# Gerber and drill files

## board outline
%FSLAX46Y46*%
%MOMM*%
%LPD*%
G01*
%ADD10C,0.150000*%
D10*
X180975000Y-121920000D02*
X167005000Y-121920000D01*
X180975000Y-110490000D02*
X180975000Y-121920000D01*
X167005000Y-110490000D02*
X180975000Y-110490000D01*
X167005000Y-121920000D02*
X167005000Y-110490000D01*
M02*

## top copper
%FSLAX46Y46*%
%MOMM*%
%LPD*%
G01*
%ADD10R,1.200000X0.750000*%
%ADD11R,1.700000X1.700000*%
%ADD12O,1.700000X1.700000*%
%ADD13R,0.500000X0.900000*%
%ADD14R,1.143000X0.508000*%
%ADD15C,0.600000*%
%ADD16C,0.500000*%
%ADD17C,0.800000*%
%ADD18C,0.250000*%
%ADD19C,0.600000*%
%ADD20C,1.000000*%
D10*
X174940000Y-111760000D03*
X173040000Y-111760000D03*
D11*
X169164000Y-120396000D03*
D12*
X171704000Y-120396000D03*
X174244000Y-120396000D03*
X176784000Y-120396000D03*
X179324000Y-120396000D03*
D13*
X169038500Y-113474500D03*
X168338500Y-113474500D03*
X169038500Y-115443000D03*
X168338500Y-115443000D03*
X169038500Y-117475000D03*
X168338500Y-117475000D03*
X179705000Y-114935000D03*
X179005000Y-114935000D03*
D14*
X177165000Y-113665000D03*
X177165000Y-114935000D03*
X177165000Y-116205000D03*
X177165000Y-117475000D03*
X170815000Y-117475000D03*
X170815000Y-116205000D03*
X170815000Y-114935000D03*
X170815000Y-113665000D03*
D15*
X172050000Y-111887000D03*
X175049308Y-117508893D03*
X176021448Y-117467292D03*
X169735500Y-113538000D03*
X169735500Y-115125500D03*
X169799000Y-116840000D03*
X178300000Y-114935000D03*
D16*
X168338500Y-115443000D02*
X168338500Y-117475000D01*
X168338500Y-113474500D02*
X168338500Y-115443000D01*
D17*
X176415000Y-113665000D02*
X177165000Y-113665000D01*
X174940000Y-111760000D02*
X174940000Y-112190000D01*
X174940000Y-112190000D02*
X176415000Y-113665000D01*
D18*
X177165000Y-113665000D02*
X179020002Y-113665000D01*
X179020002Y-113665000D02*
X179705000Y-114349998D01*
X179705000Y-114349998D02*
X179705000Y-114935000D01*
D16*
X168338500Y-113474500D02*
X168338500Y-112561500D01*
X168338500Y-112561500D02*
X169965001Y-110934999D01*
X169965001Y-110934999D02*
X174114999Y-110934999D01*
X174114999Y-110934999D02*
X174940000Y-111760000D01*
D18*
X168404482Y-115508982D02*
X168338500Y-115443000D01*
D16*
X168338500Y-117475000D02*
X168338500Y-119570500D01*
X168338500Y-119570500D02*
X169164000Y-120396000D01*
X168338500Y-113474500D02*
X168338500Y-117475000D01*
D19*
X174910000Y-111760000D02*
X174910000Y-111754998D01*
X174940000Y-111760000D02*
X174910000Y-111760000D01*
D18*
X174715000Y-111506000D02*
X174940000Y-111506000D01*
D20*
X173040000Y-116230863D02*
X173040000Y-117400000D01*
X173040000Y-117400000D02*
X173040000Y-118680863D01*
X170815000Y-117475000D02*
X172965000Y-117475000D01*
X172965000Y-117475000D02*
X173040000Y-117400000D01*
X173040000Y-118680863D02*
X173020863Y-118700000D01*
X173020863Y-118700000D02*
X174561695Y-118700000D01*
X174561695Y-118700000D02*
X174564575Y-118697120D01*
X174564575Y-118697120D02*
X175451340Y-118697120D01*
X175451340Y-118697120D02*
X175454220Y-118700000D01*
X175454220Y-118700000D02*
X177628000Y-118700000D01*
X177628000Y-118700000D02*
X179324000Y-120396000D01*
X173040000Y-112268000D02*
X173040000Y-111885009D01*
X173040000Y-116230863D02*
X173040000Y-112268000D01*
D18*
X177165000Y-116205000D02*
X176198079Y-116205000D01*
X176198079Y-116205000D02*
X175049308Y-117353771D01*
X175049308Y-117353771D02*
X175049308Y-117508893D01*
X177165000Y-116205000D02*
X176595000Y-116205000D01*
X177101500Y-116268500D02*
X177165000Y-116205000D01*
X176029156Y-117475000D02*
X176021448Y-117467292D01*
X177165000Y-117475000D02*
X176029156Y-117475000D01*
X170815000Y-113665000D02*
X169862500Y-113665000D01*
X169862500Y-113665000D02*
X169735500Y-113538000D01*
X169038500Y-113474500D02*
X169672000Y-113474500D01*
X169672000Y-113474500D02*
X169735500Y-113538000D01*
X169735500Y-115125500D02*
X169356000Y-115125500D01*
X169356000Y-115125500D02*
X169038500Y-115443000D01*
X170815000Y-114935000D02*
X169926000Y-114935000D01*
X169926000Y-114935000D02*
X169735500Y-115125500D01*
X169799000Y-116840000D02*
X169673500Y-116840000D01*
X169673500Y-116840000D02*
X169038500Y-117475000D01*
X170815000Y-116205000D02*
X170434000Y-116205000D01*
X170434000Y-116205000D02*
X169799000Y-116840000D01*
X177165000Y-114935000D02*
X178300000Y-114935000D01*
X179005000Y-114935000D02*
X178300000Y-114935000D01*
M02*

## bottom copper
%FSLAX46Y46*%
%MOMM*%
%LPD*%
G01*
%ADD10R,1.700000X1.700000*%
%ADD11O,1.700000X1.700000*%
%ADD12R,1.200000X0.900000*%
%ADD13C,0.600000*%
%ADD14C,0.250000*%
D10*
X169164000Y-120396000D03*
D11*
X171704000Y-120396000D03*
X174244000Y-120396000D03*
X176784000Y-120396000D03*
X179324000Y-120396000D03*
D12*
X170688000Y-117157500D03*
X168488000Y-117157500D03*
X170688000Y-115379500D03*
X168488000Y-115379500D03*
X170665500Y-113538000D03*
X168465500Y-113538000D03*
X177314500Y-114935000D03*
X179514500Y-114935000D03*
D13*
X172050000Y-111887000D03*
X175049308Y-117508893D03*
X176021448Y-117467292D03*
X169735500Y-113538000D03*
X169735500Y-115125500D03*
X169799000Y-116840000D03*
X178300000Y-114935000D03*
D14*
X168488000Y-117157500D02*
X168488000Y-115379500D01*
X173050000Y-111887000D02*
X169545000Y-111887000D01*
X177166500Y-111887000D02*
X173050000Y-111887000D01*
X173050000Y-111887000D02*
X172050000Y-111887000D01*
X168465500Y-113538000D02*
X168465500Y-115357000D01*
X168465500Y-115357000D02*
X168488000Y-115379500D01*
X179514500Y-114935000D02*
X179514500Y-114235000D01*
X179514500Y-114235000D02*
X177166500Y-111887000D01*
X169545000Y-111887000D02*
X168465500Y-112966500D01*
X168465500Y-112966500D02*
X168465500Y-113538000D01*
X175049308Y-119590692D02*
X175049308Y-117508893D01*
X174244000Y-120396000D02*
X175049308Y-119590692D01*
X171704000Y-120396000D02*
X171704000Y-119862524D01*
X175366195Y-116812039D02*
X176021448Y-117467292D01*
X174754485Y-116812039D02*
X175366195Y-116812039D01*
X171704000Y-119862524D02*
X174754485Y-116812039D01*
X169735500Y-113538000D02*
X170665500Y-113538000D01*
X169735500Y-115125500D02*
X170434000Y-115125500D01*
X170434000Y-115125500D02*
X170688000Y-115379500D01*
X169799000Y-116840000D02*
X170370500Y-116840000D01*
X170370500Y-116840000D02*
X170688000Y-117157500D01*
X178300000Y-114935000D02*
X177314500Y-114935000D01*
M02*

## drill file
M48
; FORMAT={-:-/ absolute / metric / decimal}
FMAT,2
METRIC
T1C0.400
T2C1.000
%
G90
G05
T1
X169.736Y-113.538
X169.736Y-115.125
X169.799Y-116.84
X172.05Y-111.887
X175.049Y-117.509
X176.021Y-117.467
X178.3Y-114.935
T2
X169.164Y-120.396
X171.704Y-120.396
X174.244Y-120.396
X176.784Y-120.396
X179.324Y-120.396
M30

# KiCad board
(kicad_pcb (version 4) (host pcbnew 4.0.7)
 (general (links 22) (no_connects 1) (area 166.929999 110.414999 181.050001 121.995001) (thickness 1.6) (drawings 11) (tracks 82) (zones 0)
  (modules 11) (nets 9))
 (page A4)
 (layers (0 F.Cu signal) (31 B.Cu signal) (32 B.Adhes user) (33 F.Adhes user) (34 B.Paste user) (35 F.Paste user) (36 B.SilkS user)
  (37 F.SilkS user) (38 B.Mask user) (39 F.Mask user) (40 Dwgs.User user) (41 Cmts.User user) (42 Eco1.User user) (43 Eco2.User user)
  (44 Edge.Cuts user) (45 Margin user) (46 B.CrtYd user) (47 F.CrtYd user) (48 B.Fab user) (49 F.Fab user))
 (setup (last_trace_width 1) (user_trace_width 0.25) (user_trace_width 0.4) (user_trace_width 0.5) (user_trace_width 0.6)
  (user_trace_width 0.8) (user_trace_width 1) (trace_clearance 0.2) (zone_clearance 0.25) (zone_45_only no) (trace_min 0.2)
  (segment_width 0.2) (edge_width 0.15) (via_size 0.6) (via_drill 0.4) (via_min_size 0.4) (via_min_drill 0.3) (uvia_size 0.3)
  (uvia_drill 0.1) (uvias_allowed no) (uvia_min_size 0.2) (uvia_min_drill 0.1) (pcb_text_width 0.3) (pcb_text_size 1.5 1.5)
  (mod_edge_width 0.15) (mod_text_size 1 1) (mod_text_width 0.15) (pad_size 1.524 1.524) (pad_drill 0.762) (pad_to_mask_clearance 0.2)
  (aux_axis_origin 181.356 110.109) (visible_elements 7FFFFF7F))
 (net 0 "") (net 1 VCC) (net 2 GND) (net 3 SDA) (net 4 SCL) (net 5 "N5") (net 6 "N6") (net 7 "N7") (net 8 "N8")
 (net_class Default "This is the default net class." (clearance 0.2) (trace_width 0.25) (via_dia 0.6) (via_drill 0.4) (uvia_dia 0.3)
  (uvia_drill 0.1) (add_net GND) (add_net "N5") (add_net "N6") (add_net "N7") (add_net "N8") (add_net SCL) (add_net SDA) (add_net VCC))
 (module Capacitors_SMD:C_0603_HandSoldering (layer F.Cu) (at 173.99 111.76 180)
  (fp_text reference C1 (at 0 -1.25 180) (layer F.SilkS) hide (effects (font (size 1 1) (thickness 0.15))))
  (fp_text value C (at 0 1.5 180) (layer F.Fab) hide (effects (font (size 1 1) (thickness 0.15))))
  (pad 1 smd rect (at -0.95 0 180) (size 1.2 0.75) (layers F.Cu F.Paste F.Mask) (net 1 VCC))
  (pad 2 smd rect (at 0.95 0 180) (size 1.2 0.75) (layers F.Cu F.Paste F.Mask) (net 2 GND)))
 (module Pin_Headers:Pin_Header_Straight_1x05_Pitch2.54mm (layer F.Cu) (at 169.164 120.396 90)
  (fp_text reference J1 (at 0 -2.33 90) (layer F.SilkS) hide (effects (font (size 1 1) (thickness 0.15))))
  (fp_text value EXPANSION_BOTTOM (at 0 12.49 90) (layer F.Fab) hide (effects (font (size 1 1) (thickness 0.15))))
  (pad 1 thru_hole rect (at 0 0 90) (size 1.7 1.7) (drill 1) (layers *.Cu *.Mask) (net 1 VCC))
  (pad 2 thru_hole oval (at 0 2.54 90) (size 1.7 1.7) (drill 1) (layers *.Cu *.Mask) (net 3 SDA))
  (pad 3 thru_hole oval (at 0 5.08 90) (size 1.7 1.7) (drill 1) (layers *.Cu *.Mask) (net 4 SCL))
  (pad 4 thru_hole oval (at 0 7.62 90) (size 1.7 1.7) (drill 1) (layers *.Cu *.Mask))
  (pad 5 thru_hole oval (at 0 10.16 90) (size 1.7 1.7) (drill 1) (layers *.Cu *.Mask) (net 2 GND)))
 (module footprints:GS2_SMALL (layer F.Cu) (at 168.3385 113.4745 270)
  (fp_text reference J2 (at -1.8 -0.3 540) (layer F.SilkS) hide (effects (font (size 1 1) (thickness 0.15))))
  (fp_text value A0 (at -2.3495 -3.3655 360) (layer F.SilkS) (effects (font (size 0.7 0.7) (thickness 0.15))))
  (pad 1 smd rect (at 0 -0.7 270) (size 0.9 0.5) (layers F.Cu F.Paste F.Mask) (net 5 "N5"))
  (pad 2 smd rect (at 0 0 270) (size 0.9 0.5) (layers F.Cu F.Paste F.Mask) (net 1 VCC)))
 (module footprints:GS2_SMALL (layer F.Cu) (at 168.3385 115.443 270)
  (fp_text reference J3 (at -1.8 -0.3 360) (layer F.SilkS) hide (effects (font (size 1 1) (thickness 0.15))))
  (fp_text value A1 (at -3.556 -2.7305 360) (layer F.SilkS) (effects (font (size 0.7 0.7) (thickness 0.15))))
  (pad 1 smd rect (at 0 -0.7 270) (size 0.9 0.5) (layers F.Cu F.Paste F.Mask) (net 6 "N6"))
  (pad 2 smd rect (at 0 0 270) (size 0.9 0.5) (layers F.Cu F.Paste F.Mask) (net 1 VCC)))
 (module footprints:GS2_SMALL (layer F.Cu) (at 168.3385 117.475 270)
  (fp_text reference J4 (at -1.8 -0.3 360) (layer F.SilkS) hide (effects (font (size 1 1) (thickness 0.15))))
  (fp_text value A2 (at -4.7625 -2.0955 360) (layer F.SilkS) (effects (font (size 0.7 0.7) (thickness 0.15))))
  (pad 1 smd rect (at 0 -0.7 270) (size 0.9 0.5) (layers F.Cu F.Paste F.Mask) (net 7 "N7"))
  (pad 2 smd rect (at 0 0 270) (size 0.9 0.5) (layers F.Cu F.Paste F.Mask) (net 1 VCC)))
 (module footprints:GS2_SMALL (layer F.Cu) (at 179.005 114.935 270)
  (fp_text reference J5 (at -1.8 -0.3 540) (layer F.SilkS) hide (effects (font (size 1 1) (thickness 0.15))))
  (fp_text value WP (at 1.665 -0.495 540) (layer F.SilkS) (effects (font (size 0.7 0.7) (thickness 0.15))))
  (pad 1 smd rect (at 0 -0.7 270) (size 0.9 0.5) (layers F.Cu F.Paste F.Mask) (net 1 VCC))
  (pad 2 smd rect (at 0 0 270) (size 0.9 0.5) (layers F.Cu F.Paste F.Mask) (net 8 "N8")))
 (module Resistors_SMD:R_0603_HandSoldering (layer B.Cu) (at 169.588 117.1575 180)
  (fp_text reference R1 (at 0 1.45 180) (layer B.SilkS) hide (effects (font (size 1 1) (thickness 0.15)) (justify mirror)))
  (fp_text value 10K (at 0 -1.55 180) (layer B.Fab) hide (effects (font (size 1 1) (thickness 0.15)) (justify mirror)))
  (pad 1 smd rect (at -1.1 0 180) (size 1.2 0.9) (layers B.Cu B.Paste B.Mask) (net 7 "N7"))
  (pad 2 smd rect (at 1.1 0 180) (size 1.2 0.9) (layers B.Cu B.Paste B.Mask) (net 2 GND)))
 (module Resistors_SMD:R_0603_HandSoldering (layer B.Cu) (at 169.588 115.3795 180)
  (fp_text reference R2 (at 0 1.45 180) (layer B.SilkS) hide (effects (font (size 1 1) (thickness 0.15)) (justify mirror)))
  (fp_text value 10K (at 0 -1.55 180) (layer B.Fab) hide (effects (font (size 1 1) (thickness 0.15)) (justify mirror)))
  (pad 1 smd rect (at -1.1 0 180) (size 1.2 0.9) (layers B.Cu B.Paste B.Mask) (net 6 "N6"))
  (pad 2 smd rect (at 1.1 0 180) (size 1.2 0.9) (layers B.Cu B.Paste B.Mask) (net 2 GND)))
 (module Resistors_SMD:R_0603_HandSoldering (layer B.Cu) (at 169.5655 113.538 180)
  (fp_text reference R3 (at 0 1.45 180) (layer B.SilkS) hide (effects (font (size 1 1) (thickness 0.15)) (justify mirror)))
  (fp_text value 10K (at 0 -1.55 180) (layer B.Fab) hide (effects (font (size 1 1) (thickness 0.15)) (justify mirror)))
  (pad 1 smd rect (at -1.1 0 180) (size 1.2 0.9) (layers B.Cu B.Paste B.Mask) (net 5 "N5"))
  (pad 2 smd rect (at 1.1 0 180) (size 1.2 0.9) (layers B.Cu B.Paste B.Mask) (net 2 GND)))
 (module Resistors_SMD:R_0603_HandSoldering (layer B.Cu) (at 178.4145 114.935)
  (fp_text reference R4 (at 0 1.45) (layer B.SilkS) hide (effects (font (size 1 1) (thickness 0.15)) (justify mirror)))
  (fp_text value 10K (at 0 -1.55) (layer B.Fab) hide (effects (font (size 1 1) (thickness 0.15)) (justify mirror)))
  (pad 1 smd rect (at -1.1 0) (size 1.2 0.9) (layers B.Cu B.Paste B.Mask) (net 8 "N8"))
  (pad 2 smd rect (at 1.1 0) (size 1.2 0.9) (layers B.Cu B.Paste B.Mask) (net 2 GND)))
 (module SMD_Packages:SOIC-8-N (layer F.Cu) (at 173.99 115.57 270)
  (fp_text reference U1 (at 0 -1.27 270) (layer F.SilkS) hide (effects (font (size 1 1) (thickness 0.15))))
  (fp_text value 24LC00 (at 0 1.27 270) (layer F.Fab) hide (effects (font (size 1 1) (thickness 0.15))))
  (pad 8 smd rect (at -1.905 -3.175 270) (size 0.508 1.143) (layers F.Cu F.Paste F.Mask) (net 1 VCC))
  (pad 7 smd rect (at -0.635 -3.175 270) (size 0.508 1.143) (layers F.Cu F.Paste F.Mask) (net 8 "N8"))
  (pad 6 smd rect (at 0.635 -3.175 270) (size 0.508 1.143) (layers F.Cu F.Paste F.Mask) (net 4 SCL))
  (pad 5 smd rect (at 1.905 -3.175 270) (size 0.508 1.143) (layers F.Cu F.Paste F.Mask) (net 3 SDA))
  (pad 4 smd rect (at 1.905 3.175 270) (size 0.508 1.143) (layers F.Cu F.Paste F.Mask) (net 2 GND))
  (pad 3 smd rect (at 0.635 3.175 270) (size 0.508 1.143) (layers F.Cu F.Paste F.Mask) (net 7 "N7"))
  (pad 2 smd rect (at -0.635 3.175 270) (size 0.508 1.143) (layers F.Cu F.Paste F.Mask) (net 6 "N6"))
  (pad 1 smd rect (at -1.905 3.175 270) (size 0.508 1.143) (layers F.Cu F.Paste F.Mask) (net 5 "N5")))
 (gr_line (start 180.975 121.92) (end 167.005 121.92) (layer Edge.Cuts) (width 0.15))
 (gr_line (start 180.975 110.49) (end 180.975 121.92) (layer Edge.Cuts) (width 0.15))
 (gr_line (start 167.005 110.49) (end 180.975 110.49) (layer Edge.Cuts) (width 0.15))
 (gr_line (start 167.005 121.92) (end 167.005 110.49) (layer Edge.Cuts) (width 0.15))
 (segment (start 168.3385 115.443) (end 168.3385 117.475) (width 0.5) (layer F.Cu) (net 1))
 (segment (start 168.3385 113.4745) (end 168.3385 115.443) (width 0.5) (layer F.Cu) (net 1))
 (segment (start 176.415 113.665) (end 177.165 113.665) (width 0.8) (layer F.Cu) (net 1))
 (segment (start 174.94 111.76) (end 174.94 112.19) (width 0.8) (layer F.Cu) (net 1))
 (segment (start 174.94 112.19) (end 176.415 113.665) (width 0.8) (layer F.Cu) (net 1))
 (segment (start 177.165 113.665) (end 179.020002 113.665) (width 0.25) (layer F.Cu) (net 1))
 (segment (start 179.020002 113.665) (end 179.705 114.349998) (width 0.25) (layer F.Cu) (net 1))
 (segment (start 179.705 114.349998) (end 179.705 114.935) (width 0.25) (layer F.Cu) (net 1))
 (segment (start 168.3385 113.4745) (end 168.3385 112.5615) (width 0.5) (layer F.Cu) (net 1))
 (segment (start 168.3385 112.5615) (end 169.965001 110.934999) (width 0.5) (layer F.Cu) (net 1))
 (segment (start 169.965001 110.934999) (end 174.114999 110.934999) (width 0.5) (layer F.Cu) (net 1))
 (segment (start 174.114999 110.934999) (end 174.94 111.76) (width 0.5) (layer F.Cu) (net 1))
 (segment (start 168.404482 115.508982) (end 168.3385 115.443) (width 0.25) (layer F.Cu) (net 1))
 (segment (start 168.3385 117.475) (end 168.3385 119.5705) (width 0.5) (layer F.Cu) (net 1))
 (segment (start 168.3385 119.5705) (end 169.164 120.396) (width 0.5) (layer F.Cu) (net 1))
 (segment (start 168.3385 113.4745) (end 168.3385 117.475) (width 0.5) (layer F.Cu) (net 1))
 (segment (start 174.91 111.76) (end 174.91 111.754998) (width 0.6) (layer F.Cu) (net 1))
 (segment (start 174.94 111.76) (end 174.91 111.76) (width 0.6) (layer F.Cu) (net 1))
 (segment (start 174.715 111.506) (end 174.94 111.506) (width 0.25) (layer F.Cu) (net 1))
 (segment (start 173.04 116.230863) (end 173.04 117.4) (width 1) (layer F.Cu) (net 2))
 (segment (start 173.04 117.4) (end 173.04 118.680863) (width 1) (layer F.Cu) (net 2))
 (segment (start 170.815 117.475) (end 172.965 117.475) (width 1) (layer F.Cu) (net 2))
 (segment (start 172.965 117.475) (end 173.04 117.4) (width 1) (layer F.Cu) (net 2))
 (segment (start 173.04 118.680863) (end 173.020863 118.7) (width 1) (layer F.Cu) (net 2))
 (segment (start 173.020863 118.7) (end 174.561695 118.7) (width 1) (layer F.Cu) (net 2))
 (segment (start 174.561695 118.7) (end 174.564575 118.69712) (width 1) (layer F.Cu) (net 2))
 (segment (start 174.564575 118.69712) (end 175.45134 118.69712) (width 1) (layer F.Cu) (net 2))
 (segment (start 175.45134 118.69712) (end 175.45422 118.7) (width 1) (layer F.Cu) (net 2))
 (segment (start 175.45422 118.7) (end 177.628 118.7) (width 1) (layer F.Cu) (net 2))
 (segment (start 177.628 118.7) (end 179.324 120.396) (width 1) (layer F.Cu) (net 2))
 (segment (start 168.488 117.1575) (end 168.488 115.3795) (width 0.25) (layer B.Cu) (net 2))
 (segment (start 173.05 111.887) (end 169.545 111.887) (width 0.25) (layer B.Cu) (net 2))
 (segment (start 177.1665 111.887) (end 173.05 111.887) (width 0.25) (layer B.Cu) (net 2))
 (segment (start 173.05 111.887) (end 172.05 111.887) (width 0.25) (layer B.Cu) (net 2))
 (via (at 172.05 111.887) (size 0.6) (drill 0.4) (layers F.Cu B.Cu) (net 2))
 (segment (start 173.04 112.268) (end 173.04 111.885009) (width 1) (layer F.Cu) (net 2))
 (segment (start 173.04 116.230863) (end 173.04 112.268) (width 1) (layer F.Cu) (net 2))
 (segment (start 168.4655 113.538) (end 168.4655 115.357) (width 0.25) (layer B.Cu) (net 2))
 (segment (start 168.4655 115.357) (end 168.488 115.3795) (width 0.25) (layer B.Cu) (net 2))
 (segment (start 179.5145 114.935) (end 179.5145 114.235) (width 0.25) (layer B.Cu) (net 2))
 (segment (start 179.5145 114.235) (end 177.1665 111.887) (width 0.25) (layer B.Cu) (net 2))
 (segment (start 169.545 111.887) (end 168.4655 112.9665) (width 0.25) (layer B.Cu) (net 2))
 (segment (start 168.4655 112.9665) (end 168.4655 113.538) (width 0.25) (layer B.Cu) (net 2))
 (segment (start 177.165 116.205) (end 176.198079 116.205) (width 0.25) (layer F.Cu) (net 4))
 (segment (start 176.198079 116.205) (end 175.049308 117.353771) (width 0.25) (layer F.Cu) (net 4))
 (segment (start 175.049308 117.353771) (end 175.049308 117.508893) (width 0.25) (layer F.Cu) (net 4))
 (segment (start 175.049308 119.590692) (end 175.049308 117.508893) (width 0.25) (layer B.Cu) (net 4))
 (via (at 175.049308 117.508893) (size 0.6) (drill 0.4) (layers F.Cu B.Cu) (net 4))
 (segment (start 174.244 120.396) (end 175.049308 119.590692) (width 0.25) (layer B.Cu) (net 4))
 (segment (start 177.165 116.205) (end 176.595 116.205) (width 0.25) (layer F.Cu) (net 4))
 (segment (start 177.1015 116.2685) (end 177.165 116.205) (width 0.25) (layer F.Cu) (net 4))
 (segment (start 171.704 120.396) (end 171.704 119.862524) (width 0.25) (layer B.Cu) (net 3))
 (segment (start 176.029156 117.475) (end 176.021448 117.467292) (width 0.25) (layer F.Cu) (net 3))
 (segment (start 177.165 117.475) (end 176.029156 117.475) (width 0.25) (layer F.Cu) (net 3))
 (segment (start 175.366195 116.812039) (end 176.021448 117.467292) (width 0.25) (layer B.Cu) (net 3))
 (segment (start 174.754485 116.812039) (end 175.366195 116.812039) (width 0.25) (layer B.Cu) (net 3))
 (segment (start 171.704 119.862524) (end 174.754485 116.812039) (width 0.25) (layer B.Cu) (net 3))
 (via (at 176.021448 117.467292) (size 0.6) (drill 0.4) (layers F.Cu B.Cu) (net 3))
 (segment (start 170.815 113.665) (end 169.8625 113.665) (width 0.25) (layer F.Cu) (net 5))
 (segment (start 169.8625 113.665) (end 169.7355 113.538) (width 0.25) (layer F.Cu) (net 5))
 (segment (start 169.7355 113.538) (end 170.6655 113.538) (width 0.25) (layer B.Cu) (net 5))
 (segment (start 169.0385 113.4745) (end 169.672 113.4745) (width 0.25) (layer F.Cu) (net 5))
 (segment (start 169.672 113.4745) (end 169.7355 113.538) (width 0.25) (layer F.Cu) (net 5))
 (via (at 169.7355 113.538) (size 0.6) (drill 0.4) (layers F.Cu B.Cu) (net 5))
 (segment (start 169.7355 115.1255) (end 169.356 115.1255) (width 0.25) (layer F.Cu) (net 6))
 (segment (start 169.356 115.1255) (end 169.0385 115.443) (width 0.25) (layer F.Cu) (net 6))
 (segment (start 169.7355 115.1255) (end 170.434 115.1255) (width 0.25) (layer B.Cu) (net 6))
 (segment (start 170.434 115.1255) (end 170.688 115.3795) (width 0.25) (layer B.Cu) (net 6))
 (segment (start 170.815 114.935) (end 169.926 114.935) (width 0.25) (layer F.Cu) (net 6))
 (segment (start 169.926 114.935) (end 169.7355 115.1255) (width 0.25) (layer F.Cu) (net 6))
 (via (at 169.7355 115.1255) (size 0.6) (drill 0.4) (layers F.Cu B.Cu) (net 6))
 (segment (start 169.799 116.84) (end 169.6735 116.84) (width 0.25) (layer F.Cu) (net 7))
 (segment (start 169.6735 116.84) (end 169.0385 117.475) (width 0.25) (layer F.Cu) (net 7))
 (segment (start 169.799 116.84) (end 170.3705 116.84) (width 0.25) (layer B.Cu) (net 7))
 (segment (start 170.3705 116.84) (end 170.688 117.1575) (width 0.25) (layer B.Cu) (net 7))
 (segment (start 170.815 116.205) (end 170.434 116.205) (width 0.25) (layer F.Cu) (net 7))
 (segment (start 170.434 116.205) (end 169.799 116.84) (width 0.25) (layer F.Cu) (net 7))
 (via (at 169.799 116.84) (size 0.6) (drill 0.4) (layers F.Cu B.Cu) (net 7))
 (segment (start 178.3 114.935) (end 177.3145 114.935) (width 0.25) (layer B.Cu) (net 8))
 (segment (start 177.165 114.935) (end 178.3 114.935) (width 0.25) (layer F.Cu) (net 8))
 (segment (start 179.005 114.935) (end 178.3 114.935) (width 0.25) (layer F.Cu) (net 8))
 (via (at 178.3 114.935) (size 0.6) (drill 0.4) (layers F.Cu B.Cu) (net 8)))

